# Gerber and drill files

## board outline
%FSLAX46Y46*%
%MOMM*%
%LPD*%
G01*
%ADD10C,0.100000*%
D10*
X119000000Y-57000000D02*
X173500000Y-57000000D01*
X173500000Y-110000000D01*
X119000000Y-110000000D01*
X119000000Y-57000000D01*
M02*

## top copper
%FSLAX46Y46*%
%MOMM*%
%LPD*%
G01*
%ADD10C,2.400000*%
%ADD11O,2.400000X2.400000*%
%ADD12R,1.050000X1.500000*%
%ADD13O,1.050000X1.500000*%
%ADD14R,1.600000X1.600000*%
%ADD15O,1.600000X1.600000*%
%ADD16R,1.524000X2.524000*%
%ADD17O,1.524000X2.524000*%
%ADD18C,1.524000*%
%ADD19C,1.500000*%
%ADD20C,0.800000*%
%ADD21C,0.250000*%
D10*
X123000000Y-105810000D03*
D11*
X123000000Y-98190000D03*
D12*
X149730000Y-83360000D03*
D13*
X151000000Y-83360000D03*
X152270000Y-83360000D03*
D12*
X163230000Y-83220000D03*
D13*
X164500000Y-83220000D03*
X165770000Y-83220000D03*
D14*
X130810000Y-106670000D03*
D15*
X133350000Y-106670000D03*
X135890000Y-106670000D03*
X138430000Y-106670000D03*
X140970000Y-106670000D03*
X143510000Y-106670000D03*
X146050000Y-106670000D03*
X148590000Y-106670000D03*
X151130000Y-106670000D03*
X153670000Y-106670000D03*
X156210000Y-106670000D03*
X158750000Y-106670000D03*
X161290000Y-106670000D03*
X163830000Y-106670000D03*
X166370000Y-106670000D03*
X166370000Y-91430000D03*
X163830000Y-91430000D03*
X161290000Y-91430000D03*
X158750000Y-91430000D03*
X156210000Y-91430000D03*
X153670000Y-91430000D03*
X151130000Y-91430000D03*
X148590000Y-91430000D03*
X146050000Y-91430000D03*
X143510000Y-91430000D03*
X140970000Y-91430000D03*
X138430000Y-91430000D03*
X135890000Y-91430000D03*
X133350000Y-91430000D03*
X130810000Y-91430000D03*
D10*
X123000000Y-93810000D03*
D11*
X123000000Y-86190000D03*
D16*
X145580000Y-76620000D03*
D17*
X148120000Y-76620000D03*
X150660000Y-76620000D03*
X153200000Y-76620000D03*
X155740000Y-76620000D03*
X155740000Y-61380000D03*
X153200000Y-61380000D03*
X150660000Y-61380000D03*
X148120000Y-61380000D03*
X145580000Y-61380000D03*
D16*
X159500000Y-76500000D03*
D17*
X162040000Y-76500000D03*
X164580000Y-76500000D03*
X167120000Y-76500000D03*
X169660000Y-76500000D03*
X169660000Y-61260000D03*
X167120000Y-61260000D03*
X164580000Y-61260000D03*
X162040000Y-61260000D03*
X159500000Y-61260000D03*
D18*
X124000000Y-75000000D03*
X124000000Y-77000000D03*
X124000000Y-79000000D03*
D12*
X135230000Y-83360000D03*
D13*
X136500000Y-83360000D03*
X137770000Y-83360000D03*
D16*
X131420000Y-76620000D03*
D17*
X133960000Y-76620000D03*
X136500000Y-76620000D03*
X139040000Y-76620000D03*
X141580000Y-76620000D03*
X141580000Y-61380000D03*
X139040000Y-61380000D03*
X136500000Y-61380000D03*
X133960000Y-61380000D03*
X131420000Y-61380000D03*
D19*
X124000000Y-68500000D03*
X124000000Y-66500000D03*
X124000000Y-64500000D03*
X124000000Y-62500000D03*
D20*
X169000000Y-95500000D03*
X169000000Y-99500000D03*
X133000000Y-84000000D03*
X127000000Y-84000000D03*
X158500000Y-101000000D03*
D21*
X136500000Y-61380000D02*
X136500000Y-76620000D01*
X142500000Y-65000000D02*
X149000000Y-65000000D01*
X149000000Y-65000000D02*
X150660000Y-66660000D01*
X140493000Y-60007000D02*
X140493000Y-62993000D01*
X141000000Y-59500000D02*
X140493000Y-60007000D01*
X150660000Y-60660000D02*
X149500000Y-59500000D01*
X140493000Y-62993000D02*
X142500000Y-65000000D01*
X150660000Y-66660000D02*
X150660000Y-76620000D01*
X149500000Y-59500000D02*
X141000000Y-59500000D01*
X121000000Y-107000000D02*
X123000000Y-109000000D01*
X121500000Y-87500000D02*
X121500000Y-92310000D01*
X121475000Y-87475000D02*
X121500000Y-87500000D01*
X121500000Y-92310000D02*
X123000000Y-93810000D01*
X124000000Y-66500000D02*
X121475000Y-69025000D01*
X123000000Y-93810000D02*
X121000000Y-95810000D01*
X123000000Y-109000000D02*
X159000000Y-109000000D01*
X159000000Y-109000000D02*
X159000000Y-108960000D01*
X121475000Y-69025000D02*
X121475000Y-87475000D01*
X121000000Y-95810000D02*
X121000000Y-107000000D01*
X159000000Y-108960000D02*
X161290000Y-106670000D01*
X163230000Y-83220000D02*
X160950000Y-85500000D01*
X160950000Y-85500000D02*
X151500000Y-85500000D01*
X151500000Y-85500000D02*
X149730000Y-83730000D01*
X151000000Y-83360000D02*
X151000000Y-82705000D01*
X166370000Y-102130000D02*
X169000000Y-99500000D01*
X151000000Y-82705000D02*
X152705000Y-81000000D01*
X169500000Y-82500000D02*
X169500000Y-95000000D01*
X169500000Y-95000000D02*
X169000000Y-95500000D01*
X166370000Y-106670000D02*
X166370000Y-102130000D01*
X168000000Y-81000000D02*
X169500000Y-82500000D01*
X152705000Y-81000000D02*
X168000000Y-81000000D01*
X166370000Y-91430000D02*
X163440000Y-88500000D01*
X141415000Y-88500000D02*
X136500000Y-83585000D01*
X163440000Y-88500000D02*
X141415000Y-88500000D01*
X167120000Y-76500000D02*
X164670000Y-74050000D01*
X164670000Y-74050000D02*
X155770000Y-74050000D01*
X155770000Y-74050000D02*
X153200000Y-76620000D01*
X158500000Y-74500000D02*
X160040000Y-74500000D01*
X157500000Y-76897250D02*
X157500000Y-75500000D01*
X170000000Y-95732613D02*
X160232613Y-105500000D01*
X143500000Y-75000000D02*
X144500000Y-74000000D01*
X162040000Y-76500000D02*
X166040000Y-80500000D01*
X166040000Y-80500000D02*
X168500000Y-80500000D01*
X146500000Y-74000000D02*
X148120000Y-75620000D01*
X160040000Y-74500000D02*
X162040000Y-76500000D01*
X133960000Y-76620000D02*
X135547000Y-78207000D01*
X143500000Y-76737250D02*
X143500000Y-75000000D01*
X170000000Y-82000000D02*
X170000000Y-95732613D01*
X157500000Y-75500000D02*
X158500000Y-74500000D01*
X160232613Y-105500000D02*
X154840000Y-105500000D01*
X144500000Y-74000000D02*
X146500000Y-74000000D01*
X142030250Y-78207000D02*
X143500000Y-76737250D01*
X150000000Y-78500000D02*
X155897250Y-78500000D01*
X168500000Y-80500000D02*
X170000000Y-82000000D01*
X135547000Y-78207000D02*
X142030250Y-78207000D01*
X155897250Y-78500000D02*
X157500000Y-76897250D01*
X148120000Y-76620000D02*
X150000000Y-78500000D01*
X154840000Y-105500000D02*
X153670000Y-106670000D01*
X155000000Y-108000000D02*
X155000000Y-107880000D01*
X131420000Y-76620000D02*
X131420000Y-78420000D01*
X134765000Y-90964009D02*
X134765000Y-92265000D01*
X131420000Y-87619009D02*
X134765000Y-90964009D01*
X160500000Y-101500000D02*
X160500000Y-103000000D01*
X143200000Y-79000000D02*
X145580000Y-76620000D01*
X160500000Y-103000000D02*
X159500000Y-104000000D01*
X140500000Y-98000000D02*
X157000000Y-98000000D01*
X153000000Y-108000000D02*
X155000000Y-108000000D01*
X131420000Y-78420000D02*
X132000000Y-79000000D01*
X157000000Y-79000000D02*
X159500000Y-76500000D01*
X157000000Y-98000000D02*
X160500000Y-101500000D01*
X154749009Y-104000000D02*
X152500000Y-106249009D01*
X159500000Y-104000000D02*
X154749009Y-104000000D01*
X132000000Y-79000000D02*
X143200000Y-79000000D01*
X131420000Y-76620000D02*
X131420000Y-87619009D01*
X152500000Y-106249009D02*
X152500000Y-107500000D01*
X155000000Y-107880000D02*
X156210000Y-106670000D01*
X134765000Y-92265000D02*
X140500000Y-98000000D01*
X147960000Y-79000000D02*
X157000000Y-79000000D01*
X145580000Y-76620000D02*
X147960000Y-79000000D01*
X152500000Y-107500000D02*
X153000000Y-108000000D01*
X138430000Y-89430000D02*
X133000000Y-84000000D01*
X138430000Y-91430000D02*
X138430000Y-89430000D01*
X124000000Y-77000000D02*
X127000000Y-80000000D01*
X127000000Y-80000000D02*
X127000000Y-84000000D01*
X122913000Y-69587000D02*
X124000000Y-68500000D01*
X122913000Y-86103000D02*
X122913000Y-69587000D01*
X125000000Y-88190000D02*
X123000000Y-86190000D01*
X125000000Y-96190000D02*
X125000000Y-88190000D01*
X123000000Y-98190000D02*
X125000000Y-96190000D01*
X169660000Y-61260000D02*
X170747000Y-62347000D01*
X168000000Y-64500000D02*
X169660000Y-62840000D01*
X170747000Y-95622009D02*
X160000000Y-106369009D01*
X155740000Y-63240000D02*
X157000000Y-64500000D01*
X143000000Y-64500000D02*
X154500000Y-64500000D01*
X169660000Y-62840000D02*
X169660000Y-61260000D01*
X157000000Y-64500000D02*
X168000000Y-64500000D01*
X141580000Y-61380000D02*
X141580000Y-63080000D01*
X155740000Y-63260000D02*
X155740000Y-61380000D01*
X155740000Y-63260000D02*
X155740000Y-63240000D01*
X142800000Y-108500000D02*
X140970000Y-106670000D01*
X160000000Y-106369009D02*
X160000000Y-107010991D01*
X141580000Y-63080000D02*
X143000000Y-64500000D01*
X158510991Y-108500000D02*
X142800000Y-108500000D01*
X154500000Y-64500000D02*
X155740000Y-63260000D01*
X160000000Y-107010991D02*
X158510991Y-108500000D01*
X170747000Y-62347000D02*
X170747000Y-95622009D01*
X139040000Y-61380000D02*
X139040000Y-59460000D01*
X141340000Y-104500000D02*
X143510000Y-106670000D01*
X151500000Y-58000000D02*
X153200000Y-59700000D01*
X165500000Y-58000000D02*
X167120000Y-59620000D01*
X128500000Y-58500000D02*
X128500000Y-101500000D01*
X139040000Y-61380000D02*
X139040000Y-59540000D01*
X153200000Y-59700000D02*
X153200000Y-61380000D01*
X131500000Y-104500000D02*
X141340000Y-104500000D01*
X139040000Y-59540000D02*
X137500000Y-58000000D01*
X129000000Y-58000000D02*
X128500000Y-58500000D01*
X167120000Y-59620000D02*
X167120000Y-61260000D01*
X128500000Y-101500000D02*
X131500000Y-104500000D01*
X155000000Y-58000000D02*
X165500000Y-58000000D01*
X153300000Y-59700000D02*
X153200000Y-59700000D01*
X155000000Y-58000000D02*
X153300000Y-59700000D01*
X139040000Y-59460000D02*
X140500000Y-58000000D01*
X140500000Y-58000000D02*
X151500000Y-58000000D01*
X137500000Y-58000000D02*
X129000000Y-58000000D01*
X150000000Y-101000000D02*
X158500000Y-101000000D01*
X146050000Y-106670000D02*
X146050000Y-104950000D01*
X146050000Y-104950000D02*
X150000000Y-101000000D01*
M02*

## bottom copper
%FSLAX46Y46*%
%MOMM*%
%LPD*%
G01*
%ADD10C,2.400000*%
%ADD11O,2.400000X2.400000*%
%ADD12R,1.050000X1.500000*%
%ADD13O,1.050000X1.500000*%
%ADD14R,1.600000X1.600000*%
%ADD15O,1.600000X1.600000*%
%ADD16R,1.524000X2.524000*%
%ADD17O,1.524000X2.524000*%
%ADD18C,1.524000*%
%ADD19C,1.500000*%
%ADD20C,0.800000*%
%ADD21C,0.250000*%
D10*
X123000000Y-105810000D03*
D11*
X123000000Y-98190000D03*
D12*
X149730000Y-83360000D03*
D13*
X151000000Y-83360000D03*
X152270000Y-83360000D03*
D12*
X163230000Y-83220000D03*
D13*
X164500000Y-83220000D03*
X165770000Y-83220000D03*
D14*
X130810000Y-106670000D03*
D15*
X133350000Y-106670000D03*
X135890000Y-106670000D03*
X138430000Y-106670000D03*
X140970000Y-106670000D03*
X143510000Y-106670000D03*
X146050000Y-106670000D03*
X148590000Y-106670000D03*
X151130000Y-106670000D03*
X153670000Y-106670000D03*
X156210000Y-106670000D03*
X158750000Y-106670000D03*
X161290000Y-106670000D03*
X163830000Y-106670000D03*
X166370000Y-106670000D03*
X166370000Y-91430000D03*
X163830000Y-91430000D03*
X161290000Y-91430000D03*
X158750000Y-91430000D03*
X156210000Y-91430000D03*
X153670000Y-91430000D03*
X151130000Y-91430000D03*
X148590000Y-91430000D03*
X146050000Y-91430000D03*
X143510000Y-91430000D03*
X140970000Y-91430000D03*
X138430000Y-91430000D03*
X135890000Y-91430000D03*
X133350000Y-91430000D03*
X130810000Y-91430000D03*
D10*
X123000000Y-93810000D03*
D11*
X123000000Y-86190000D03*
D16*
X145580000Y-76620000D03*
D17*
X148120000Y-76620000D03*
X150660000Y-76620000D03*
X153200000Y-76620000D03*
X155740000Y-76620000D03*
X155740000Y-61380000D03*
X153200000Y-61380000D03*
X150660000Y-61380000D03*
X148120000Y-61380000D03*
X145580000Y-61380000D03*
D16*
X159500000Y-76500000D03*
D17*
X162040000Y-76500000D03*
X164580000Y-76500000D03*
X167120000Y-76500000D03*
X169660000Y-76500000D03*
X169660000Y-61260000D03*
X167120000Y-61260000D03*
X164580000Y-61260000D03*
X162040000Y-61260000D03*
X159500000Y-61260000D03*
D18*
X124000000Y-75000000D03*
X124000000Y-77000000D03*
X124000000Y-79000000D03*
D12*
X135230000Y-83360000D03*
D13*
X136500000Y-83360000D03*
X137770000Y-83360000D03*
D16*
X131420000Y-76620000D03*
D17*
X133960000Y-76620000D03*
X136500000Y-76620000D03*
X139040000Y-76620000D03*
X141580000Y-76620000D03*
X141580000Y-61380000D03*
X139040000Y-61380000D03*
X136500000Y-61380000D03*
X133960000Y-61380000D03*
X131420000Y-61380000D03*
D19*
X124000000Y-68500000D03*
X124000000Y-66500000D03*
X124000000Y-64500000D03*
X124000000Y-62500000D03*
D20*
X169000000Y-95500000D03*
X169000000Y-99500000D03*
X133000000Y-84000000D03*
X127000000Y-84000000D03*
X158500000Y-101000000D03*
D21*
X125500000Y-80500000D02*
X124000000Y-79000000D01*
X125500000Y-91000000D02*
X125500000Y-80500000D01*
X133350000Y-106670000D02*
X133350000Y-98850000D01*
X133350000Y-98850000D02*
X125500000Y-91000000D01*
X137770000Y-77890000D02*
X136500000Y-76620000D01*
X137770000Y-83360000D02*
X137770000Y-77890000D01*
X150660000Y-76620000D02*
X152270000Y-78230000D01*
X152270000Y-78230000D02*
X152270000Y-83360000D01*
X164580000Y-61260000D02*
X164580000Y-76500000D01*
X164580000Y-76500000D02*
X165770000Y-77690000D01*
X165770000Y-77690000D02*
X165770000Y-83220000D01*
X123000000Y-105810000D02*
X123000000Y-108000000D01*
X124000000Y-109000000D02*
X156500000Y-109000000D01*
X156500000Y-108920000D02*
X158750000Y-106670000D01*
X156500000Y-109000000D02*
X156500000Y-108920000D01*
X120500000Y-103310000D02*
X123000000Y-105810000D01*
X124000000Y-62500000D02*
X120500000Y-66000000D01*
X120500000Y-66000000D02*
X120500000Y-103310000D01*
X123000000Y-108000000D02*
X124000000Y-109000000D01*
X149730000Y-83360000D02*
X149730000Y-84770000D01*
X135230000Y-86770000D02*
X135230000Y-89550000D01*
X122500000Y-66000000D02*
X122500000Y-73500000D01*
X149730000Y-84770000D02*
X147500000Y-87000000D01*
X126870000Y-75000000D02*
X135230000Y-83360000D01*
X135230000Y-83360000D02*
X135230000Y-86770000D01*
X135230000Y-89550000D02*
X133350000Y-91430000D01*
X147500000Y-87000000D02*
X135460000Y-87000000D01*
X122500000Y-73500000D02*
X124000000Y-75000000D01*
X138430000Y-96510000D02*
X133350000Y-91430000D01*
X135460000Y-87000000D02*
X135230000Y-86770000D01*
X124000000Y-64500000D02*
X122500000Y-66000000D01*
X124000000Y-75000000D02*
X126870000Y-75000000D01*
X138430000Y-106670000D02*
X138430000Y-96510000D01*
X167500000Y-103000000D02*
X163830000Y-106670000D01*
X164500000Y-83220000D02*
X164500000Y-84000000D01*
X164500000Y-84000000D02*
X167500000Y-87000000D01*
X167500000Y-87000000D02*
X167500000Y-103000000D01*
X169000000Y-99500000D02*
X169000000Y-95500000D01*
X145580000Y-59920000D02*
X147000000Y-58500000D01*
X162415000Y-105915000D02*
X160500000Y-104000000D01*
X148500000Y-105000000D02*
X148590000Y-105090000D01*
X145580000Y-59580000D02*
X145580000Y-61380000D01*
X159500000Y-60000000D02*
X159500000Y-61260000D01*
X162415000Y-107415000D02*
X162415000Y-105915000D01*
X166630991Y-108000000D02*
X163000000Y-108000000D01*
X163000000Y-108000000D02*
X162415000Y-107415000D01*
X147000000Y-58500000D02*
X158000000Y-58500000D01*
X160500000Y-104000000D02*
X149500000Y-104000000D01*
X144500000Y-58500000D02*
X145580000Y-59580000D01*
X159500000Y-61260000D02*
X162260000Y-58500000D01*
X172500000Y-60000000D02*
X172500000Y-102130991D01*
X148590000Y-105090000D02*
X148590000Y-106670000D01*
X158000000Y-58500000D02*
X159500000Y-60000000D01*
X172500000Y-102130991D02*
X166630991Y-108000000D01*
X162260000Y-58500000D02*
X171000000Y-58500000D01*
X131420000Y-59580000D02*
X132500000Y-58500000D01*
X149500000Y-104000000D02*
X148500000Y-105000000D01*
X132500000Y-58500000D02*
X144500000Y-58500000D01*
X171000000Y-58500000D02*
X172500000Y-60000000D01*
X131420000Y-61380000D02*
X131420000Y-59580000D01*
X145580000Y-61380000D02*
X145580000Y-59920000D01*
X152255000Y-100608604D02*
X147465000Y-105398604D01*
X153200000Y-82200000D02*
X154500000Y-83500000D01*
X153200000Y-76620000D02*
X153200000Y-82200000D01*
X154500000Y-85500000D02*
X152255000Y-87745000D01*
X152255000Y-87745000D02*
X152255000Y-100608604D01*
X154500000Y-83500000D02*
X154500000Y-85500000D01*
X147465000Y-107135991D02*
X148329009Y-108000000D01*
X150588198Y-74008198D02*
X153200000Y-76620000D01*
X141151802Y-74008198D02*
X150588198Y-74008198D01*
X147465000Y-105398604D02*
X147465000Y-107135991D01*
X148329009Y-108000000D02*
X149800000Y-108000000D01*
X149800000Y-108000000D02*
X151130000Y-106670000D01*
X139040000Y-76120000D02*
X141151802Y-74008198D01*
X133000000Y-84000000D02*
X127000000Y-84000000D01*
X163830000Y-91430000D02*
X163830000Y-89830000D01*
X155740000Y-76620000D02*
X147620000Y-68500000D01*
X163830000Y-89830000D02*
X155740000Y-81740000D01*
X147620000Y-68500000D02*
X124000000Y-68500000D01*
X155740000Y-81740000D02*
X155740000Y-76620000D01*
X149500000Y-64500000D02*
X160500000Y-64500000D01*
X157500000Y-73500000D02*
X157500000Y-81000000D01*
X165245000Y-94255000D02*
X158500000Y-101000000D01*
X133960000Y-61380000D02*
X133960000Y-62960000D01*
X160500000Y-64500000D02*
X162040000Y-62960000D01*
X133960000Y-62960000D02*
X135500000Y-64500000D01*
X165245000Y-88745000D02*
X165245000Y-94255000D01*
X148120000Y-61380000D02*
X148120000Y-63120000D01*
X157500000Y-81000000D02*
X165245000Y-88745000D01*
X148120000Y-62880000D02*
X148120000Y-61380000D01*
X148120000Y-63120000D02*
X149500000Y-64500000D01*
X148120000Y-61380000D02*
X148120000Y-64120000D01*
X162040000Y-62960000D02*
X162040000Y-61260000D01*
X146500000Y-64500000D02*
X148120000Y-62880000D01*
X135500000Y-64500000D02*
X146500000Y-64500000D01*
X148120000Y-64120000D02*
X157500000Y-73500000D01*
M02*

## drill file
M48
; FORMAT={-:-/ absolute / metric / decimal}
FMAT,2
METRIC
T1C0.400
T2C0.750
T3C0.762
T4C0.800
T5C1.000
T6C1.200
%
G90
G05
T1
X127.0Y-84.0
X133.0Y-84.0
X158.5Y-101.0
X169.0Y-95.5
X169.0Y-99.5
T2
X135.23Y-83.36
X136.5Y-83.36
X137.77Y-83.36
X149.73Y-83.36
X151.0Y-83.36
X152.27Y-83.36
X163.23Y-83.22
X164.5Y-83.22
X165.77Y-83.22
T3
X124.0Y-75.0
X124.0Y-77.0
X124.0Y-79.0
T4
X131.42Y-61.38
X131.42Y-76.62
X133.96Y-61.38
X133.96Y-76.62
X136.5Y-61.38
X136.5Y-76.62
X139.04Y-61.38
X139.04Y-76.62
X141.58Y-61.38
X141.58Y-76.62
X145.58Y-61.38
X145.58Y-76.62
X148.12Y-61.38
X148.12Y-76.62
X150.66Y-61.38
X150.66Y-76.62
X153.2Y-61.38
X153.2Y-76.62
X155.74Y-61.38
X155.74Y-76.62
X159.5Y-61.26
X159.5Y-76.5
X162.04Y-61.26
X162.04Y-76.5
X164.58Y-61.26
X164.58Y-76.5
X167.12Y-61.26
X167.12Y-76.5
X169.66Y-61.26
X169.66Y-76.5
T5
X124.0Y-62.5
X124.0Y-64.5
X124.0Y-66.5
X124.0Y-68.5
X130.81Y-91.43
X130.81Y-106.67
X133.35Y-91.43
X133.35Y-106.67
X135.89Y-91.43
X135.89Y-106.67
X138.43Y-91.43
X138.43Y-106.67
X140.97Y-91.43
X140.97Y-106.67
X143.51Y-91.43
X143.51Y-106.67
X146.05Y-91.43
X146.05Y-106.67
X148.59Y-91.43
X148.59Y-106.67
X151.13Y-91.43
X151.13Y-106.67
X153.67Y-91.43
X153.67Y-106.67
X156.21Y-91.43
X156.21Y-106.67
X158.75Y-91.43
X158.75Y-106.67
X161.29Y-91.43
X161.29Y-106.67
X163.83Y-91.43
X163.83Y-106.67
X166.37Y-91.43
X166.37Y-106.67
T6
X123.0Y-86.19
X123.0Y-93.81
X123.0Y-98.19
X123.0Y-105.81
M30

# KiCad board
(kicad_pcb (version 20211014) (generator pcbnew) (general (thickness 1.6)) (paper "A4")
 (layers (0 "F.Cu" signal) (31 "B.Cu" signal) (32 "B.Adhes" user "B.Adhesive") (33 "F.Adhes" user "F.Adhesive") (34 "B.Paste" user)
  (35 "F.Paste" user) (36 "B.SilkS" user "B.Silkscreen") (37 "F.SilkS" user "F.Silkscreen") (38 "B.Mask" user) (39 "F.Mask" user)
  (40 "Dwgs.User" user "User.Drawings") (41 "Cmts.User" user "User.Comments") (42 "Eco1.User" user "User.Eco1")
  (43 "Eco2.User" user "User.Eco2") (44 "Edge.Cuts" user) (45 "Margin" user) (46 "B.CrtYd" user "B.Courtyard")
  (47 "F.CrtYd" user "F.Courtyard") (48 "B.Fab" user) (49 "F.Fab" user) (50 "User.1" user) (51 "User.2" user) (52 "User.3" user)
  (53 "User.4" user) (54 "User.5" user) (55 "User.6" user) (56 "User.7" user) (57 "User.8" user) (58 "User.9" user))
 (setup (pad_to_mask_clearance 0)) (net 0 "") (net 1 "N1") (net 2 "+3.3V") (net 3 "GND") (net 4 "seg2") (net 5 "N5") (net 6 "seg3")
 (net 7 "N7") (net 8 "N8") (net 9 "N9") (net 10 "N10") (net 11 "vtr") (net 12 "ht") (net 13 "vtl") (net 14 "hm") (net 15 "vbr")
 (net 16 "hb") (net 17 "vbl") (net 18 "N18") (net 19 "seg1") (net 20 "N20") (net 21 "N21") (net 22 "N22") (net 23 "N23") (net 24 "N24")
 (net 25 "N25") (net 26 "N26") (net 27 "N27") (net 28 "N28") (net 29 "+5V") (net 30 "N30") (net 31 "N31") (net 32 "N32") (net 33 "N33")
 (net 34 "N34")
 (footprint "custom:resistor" (layer "F.Cu") (at 123 105.81 90)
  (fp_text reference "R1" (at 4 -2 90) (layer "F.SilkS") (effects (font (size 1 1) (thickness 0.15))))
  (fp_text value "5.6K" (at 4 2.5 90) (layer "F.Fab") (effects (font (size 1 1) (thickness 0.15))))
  (pad "1" thru_hole circle (at 0 0 90) (size 2.4 2.4) (drill 1.2) (layers *.Cu *.Mask) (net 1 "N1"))
  (pad "2" thru_hole oval (at 7.62 0 90) (size 2.4 2.4) (drill 1.2) (layers *.Cu *.Mask) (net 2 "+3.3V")))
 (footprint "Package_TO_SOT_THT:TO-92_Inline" (layer "F.Cu") (at 149.73 83.36)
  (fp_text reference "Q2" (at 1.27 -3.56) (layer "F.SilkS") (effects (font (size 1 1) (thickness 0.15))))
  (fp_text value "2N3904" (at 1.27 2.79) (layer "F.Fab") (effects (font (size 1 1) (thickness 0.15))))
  (pad "1" thru_hole rect (at 0 0) (size 1.05 1.5) (drill 0.75) (layers *.Cu *.Mask) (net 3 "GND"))
  (pad "2" thru_hole oval (at 1.27 0) (size 1.05 1.5) (drill 0.75) (layers *.Cu *.Mask) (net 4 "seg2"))
  (pad "3" thru_hole oval (at 2.54 0) (size 1.05 1.5) (drill 0.75) (layers *.Cu *.Mask) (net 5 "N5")))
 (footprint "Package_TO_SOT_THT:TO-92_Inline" (layer "F.Cu") (at 163.23 83.22)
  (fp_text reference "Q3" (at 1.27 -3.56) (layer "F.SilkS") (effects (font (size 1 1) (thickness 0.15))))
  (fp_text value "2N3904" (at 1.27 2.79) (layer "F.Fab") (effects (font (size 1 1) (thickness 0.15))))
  (pad "1" thru_hole rect (at 0 0) (size 1.05 1.5) (drill 0.75) (layers *.Cu *.Mask) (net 3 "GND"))
  (pad "2" thru_hole oval (at 1.27 0) (size 1.05 1.5) (drill 0.75) (layers *.Cu *.Mask) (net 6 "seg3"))
  (pad "3" thru_hole oval (at 2.54 0) (size 1.05 1.5) (drill 0.75) (layers *.Cu *.Mask) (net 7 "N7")))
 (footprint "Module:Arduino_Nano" (layer "F.Cu") (at 130.81 106.67 90)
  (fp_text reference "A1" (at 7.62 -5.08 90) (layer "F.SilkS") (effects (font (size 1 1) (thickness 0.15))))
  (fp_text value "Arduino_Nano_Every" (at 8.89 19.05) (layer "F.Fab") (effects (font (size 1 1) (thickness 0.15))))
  (pad "1" thru_hole rect (at 0 0 90) (size 1.6 1.6) (drill 1) (layers *.Cu *.Mask) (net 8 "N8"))
  (pad "2" thru_hole oval (at 0 2.54 90) (size 1.6 1.6) (drill 1) (layers *.Cu *.Mask) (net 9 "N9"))
  (pad "3" thru_hole oval (at 0 5.08 90) (size 1.6 1.6) (drill 1) (layers *.Cu *.Mask) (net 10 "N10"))
  (pad "4" thru_hole oval (at 0 7.62 90) (size 1.6 1.6) (drill 1) (layers *.Cu *.Mask) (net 3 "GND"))
  (pad "5" thru_hole oval (at 0 10.16 90) (size 1.6 1.6) (drill 1) (layers *.Cu *.Mask) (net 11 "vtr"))
  (pad "6" thru_hole oval (at 0 12.7 90) (size 1.6 1.6) (drill 1) (layers *.Cu *.Mask) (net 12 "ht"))
  (pad "7" thru_hole oval (at 0 15.24 90) (size 1.6 1.6) (drill 1) (layers *.Cu *.Mask) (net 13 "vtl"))
  (pad "8" thru_hole oval (at 0 17.78 90) (size 1.6 1.6) (drill 1) (layers *.Cu *.Mask) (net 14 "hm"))
  (pad "9" thru_hole oval (at 0 20.32 90) (size 1.6 1.6) (drill 1) (layers *.Cu *.Mask) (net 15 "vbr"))
  (pad "10" thru_hole oval (at 0 22.86 90) (size 1.6 1.6) (drill 1) (layers *.Cu *.Mask) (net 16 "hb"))
  (pad "11" thru_hole oval (at 0 25.4 90) (size 1.6 1.6) (drill 1) (layers *.Cu *.Mask) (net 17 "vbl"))
  (pad "12" thru_hole oval (at 0 27.94 90) (size 1.6 1.6) (drill 1) (layers *.Cu *.Mask) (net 1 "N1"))
  (pad "13" thru_hole oval (at 0 30.48 90) (size 1.6 1.6) (drill 1) (layers *.Cu *.Mask) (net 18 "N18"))
  (pad "14" thru_hole oval (at 0 33.02 90) (size 1.6 1.6) (drill 1) (layers *.Cu *.Mask) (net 6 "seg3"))
  (pad "15" thru_hole oval (at 0 35.56 90) (size 1.6 1.6) (drill 1) (layers *.Cu *.Mask) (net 4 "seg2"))
  (pad "16" thru_hole oval (at 15.24 35.56 90) (size 1.6 1.6) (drill 1) (layers *.Cu *.Mask) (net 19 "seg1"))
  (pad "17" thru_hole oval (at 15.24 33.02 90) (size 1.6 1.6) (drill 1) (layers *.Cu *.Mask) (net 2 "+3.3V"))
  (pad "18" thru_hole oval (at 15.24 30.48 90) (size 1.6 1.6) (drill 1) (layers *.Cu *.Mask) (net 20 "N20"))
  (pad "19" thru_hole oval (at 15.24 27.94 90) (size 1.6 1.6) (drill 1) (layers *.Cu *.Mask) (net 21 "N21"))
  (pad "20" thru_hole oval (at 15.24 25.4 90) (size 1.6 1.6) (drill 1) (layers *.Cu *.Mask) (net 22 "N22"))
  (pad "21" thru_hole oval (at 15.24 22.86 90) (size 1.6 1.6) (drill 1) (layers *.Cu *.Mask) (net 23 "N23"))
  (pad "22" thru_hole oval (at 15.24 20.32 90) (size 1.6 1.6) (drill 1) (layers *.Cu *.Mask) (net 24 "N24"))
  (pad "23" thru_hole oval (at 15.24 17.78 90) (size 1.6 1.6) (drill 1) (layers *.Cu *.Mask) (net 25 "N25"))
  (pad "24" thru_hole oval (at 15.24 15.24 90) (size 1.6 1.6) (drill 1) (layers *.Cu *.Mask) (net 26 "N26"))
  (pad "25" thru_hole oval (at 15.24 12.7 90) (size 1.6 1.6) (drill 1) (layers *.Cu *.Mask) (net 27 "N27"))
  (pad "26" thru_hole oval (at 15.24 10.16 90) (size 1.6 1.6) (drill 1) (layers *.Cu *.Mask) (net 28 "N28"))
  (pad "27" thru_hole oval (at 15.24 7.62 90) (size 1.6 1.6) (drill 1) (layers *.Cu *.Mask) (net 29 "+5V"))
  (pad "28" thru_hole oval (at 15.24 5.08 90) (size 1.6 1.6) (drill 1) (layers *.Cu *.Mask) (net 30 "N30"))
  (pad "29" thru_hole oval (at 15.24 2.54 90) (size 1.6 1.6) (drill 1) (layers *.Cu *.Mask) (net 3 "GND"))
  (pad "30" thru_hole oval (at 15.24 0 90) (size 1.6 1.6) (drill 1) (layers *.Cu *.Mask) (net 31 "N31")))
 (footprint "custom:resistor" (layer "F.Cu") (at 123 93.81 90)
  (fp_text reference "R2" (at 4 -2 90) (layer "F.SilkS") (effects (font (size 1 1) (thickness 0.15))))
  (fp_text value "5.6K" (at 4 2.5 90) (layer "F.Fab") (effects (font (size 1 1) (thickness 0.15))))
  (pad "1" thru_hole circle (at 0 0 90) (size 2.4 2.4) (drill 1.2) (layers *.Cu *.Mask) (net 18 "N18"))
  (pad "2" thru_hole oval (at 7.62 0 90) (size 2.4 2.4) (drill 1.2) (layers *.Cu *.Mask) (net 2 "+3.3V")))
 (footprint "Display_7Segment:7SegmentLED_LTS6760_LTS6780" (layer "F.Cu") (at 145.58 76.62 90)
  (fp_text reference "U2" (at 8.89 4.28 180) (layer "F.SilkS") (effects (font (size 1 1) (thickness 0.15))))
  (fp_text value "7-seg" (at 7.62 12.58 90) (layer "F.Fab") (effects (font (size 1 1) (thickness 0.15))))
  (pad "1" thru_hole rect (at 0 0) (size 1.524 2.524) (drill 0.8) (layers *.Cu *.Mask) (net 17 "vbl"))
  (pad "2" thru_hole oval (at 0 2.54) (size 1.524 2.524) (drill 0.8) (layers *.Cu *.Mask) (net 16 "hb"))
  (pad "3" thru_hole oval (at 0 5.08) (size 1.524 2.524) (drill 0.8) (layers *.Cu *.Mask) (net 5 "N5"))
  (pad "4" thru_hole oval (at 0 7.62) (size 1.524 2.524) (drill 0.8) (layers *.Cu *.Mask) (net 15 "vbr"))
  (pad "5" thru_hole oval (at 0 10.16) (size 1.524 2.524) (drill 0.8) (layers *.Cu *.Mask) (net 2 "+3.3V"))
  (pad "6" thru_hole oval (at 15.24 10.16) (size 1.524 2.524) (drill 0.8) (layers *.Cu *.Mask) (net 11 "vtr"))
  (pad "7" thru_hole oval (at 15.24 7.62) (size 1.524 2.524) (drill 0.8) (layers *.Cu *.Mask) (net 12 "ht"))
  (pad "8" thru_hole oval (at 15.24 5.08) (size 1.524 2.524) (drill 0.8) (layers *.Cu *.Mask) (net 5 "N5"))
  (pad "9" thru_hole oval (at 15.24 2.54) (size 1.524 2.524) (drill 0.8) (layers *.Cu *.Mask) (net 13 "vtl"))
  (pad "10" thru_hole oval (at 15.24 0) (size 1.524 2.524) (drill 0.8) (layers *.Cu *.Mask) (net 14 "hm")))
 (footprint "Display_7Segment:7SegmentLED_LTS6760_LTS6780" (layer "F.Cu") (at 159.5 76.5 90)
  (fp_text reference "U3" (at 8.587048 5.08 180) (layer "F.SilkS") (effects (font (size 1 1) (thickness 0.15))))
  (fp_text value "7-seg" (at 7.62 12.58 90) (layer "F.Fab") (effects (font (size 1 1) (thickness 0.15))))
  (pad "1" thru_hole rect (at 0 0) (size 1.524 2.524) (drill 0.8) (layers *.Cu *.Mask) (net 17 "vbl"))
  (pad "2" thru_hole oval (at 0 2.54) (size 1.524 2.524) (drill 0.8) (layers *.Cu *.Mask) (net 16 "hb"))
  (pad "3" thru_hole oval (at 0 5.08) (size 1.524 2.524) (drill 0.8) (layers *.Cu *.Mask) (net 7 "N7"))
  (pad "4" thru_hole oval (at 0 7.62) (size 1.524 2.524) (drill 0.8) (layers *.Cu *.Mask) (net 15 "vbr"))
  (pad "5" thru_hole oval (at 0 10.16) (size 1.524 2.524) (drill 0.8) (layers *.Cu *.Mask) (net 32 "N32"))
  (pad "6" thru_hole oval (at 15.24 10.16) (size 1.524 2.524) (drill 0.8) (layers *.Cu *.Mask) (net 11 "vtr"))
  (pad "7" thru_hole oval (at 15.24 7.62) (size 1.524 2.524) (drill 0.8) (layers *.Cu *.Mask) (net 12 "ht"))
  (pad "8" thru_hole oval (at 15.24 5.08) (size 1.524 2.524) (drill 0.8) (layers *.Cu *.Mask) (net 7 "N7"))
  (pad "9" thru_hole oval (at 15.24 2.54) (size 1.524 2.524) (drill 0.8) (layers *.Cu *.Mask) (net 13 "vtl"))
  (pad "10" thru_hole oval (at 15.24 0) (size 1.524 2.524) (drill 0.8) (layers *.Cu *.Mask) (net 14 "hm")))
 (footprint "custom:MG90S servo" (layer "F.Cu") (at 124 77 -90)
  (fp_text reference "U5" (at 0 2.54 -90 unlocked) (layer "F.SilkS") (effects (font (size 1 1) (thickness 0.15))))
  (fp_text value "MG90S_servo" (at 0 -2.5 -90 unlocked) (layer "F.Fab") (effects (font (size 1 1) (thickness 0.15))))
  (pad "1" thru_hole circle (at -2 0 270) (size 1.524 1.524) (drill 0.762) (layers *.Cu *.Mask) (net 3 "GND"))
  (pad "2" thru_hole circle (at 0 0 270) (size 1.524 1.524) (drill 0.762) (layers *.Cu *.Mask) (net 29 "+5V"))
  (pad "3" thru_hole circle (at 2 0 270) (size 1.524 1.524) (drill 0.762) (layers *.Cu *.Mask) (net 9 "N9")))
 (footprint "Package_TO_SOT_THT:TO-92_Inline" (layer "F.Cu") (at 135.23 83.36)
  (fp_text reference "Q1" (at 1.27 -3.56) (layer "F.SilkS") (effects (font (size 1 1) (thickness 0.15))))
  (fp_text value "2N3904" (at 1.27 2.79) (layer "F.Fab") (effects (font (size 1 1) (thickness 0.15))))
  (pad "1" thru_hole rect (at 0 0) (size 1.05 1.5) (drill 0.75) (layers *.Cu *.Mask) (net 3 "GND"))
  (pad "2" thru_hole oval (at 1.27 0) (size 1.05 1.5) (drill 0.75) (layers *.Cu *.Mask) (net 19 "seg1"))
  (pad "3" thru_hole oval (at 2.54 0) (size 1.05 1.5) (drill 0.75) (layers *.Cu *.Mask) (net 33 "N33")))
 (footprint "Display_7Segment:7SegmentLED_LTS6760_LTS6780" (layer "F.Cu") (at 131.42 76.62 90)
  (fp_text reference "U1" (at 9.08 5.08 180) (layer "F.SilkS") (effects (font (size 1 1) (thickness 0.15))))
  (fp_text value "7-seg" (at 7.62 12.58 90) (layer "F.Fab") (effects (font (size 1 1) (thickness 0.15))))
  (pad "1" thru_hole rect (at 0 0) (size 1.524 2.524) (drill 0.8) (layers *.Cu *.Mask) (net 17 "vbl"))
  (pad "2" thru_hole oval (at 0 2.54) (size 1.524 2.524) (drill 0.8) (layers *.Cu *.Mask) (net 16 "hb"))
  (pad "3" thru_hole oval (at 0 5.08) (size 1.524 2.524) (drill 0.8) (layers *.Cu *.Mask) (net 33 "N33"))
  (pad "4" thru_hole oval (at 0 7.62) (size 1.524 2.524) (drill 0.8) (layers *.Cu *.Mask) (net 15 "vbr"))
  (pad "5" thru_hole oval (at 0 10.16) (size 1.524 2.524) (drill 0.8) (layers *.Cu *.Mask) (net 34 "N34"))
  (pad "6" thru_hole oval (at 15.24 10.16) (size 1.524 2.524) (drill 0.8) (layers *.Cu *.Mask) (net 11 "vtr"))
  (pad "7" thru_hole oval (at 15.24 7.62) (size 1.524 2.524) (drill 0.8) (layers *.Cu *.Mask) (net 12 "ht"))
  (pad "8" thru_hole oval (at 15.24 5.08) (size 1.524 2.524) (drill 0.8) (layers *.Cu *.Mask) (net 33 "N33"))
  (pad "9" thru_hole oval (at 15.24 2.54) (size 1.524 2.524) (drill 0.8) (layers *.Cu *.Mask) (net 13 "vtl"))
  (pad "10" thru_hole oval (at 15.24 0) (size 1.524 2.524) (drill 0.8) (layers *.Cu *.Mask) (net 14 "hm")))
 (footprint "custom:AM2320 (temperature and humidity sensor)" (layer "F.Cu") (at 124 65.5 90)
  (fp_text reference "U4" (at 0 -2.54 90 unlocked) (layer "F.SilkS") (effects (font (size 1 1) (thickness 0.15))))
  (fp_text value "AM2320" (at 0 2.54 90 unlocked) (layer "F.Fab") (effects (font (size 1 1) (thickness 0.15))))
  (pad "1" thru_hole circle (at -3 0 90) (size 1.5 1.5) (drill 1) (layers *.Cu *.Mask) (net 2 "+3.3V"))
  (pad "2" thru_hole circle (at -1 0 90) (size 1.5 1.5) (drill 1) (layers *.Cu *.Mask) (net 18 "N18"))
  (pad "3" thru_hole circle (at 1 0 90) (size 1.5 1.5) (drill 1) (layers *.Cu *.Mask) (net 3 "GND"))
  (pad "4" thru_hole circle (at 3 0 90) (size 1.5 1.5) (drill 1) (layers *.Cu *.Mask) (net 1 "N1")))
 (gr_rect (start 173.5 57) (end 119 110) (layer "Edge.Cuts") (width 0.1) (fill none))
 (segment (start 125.5 80.5) (end 124 79) (width 0.25) (layer "B.Cu") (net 9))
 (segment (start 125.5 91) (end 125.5 80.5) (width 0.25) (layer "B.Cu") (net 9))
 (segment (start 133.35 106.67) (end 133.35 98.85) (width 0.25) (layer "B.Cu") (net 9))
 (segment (start 133.35 98.85) (end 125.5 91) (width 0.25) (layer "B.Cu") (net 9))
 (segment (start 136.5 61.38) (end 136.5 76.62) (width 0.25) (layer "F.Cu") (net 33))
 (segment (start 137.77 77.89) (end 136.5 76.62) (width 0.25) (layer "B.Cu") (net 33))
 (segment (start 137.77 83.36) (end 137.77 77.89) (width 0.25) (layer "B.Cu") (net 33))
 (segment (start 142.5 65) (end 149 65) (width 0.25) (layer "F.Cu") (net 5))
 (segment (start 149 65) (end 150.66 66.66) (width 0.25) (layer "F.Cu") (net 5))
 (segment (start 140.493 60.007) (end 140.493 62.993) (width 0.25) (layer "F.Cu") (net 5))
 (segment (start 141 59.5) (end 140.493 60.007) (width 0.25) (layer "F.Cu") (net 5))
 (segment (start 150.66 60.66) (end 149.5 59.5) (width 0.25) (layer "F.Cu") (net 5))
 (segment (start 140.493 62.993) (end 142.5 65) (width 0.25) (layer "F.Cu") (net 5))
 (segment (start 150.66 66.66) (end 150.66 76.62) (width 0.25) (layer "F.Cu") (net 5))
 (segment (start 149.5 59.5) (end 141 59.5) (width 0.25) (layer "F.Cu") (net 5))
 (segment (start 150.66 76.62) (end 152.27 78.23) (width 0.25) (layer "B.Cu") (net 5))
 (segment (start 152.27 78.23) (end 152.27 83.36) (width 0.25) (layer "B.Cu") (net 5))
 (segment (start 164.58 61.26) (end 164.58 76.5) (width 0.25) (layer "B.Cu") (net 7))
 (segment (start 164.58 76.5) (end 165.77 77.69) (width 0.25) (layer "B.Cu") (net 7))
 (segment (start 165.77 77.69) (end 165.77 83.22) (width 0.25) (layer "B.Cu") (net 7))
 (segment (start 123 105.81) (end 123 108) (width 0.25) (layer "B.Cu") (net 1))
 (segment (start 124 109) (end 156.5 109) (width 0.25) (layer "B.Cu") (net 1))
 (segment (start 156.5 108.92) (end 158.75 106.67) (width 0.25) (layer "B.Cu") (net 1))
 (segment (start 156.5 109) (end 156.5 108.92) (width 0.25) (layer "B.Cu") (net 1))
 (segment (start 120.5 103.31) (end 123 105.81) (width 0.25) (layer "B.Cu") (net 1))
 (segment (start 124 62.5) (end 120.5 66) (width 0.25) (layer "B.Cu") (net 1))
 (segment (start 120.5 66) (end 120.5 103.31) (width 0.25) (layer "B.Cu") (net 1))
 (segment (start 123 108) (end 124 109) (width 0.25) (layer "B.Cu") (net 1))
 (segment (start 121 107) (end 123 109) (width 0.25) (layer "F.Cu") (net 18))
 (segment (start 121.5 87.5) (end 121.5 92.31) (width 0.25) (layer "F.Cu") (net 18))
 (segment (start 121.475 87.475) (end 121.5 87.5) (width 0.25) (layer "F.Cu") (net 18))
 (segment (start 121.5 92.31) (end 123 93.81) (width 0.25) (layer "F.Cu") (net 18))
 (segment (start 124 66.5) (end 121.475 69.025) (width 0.25) (layer "F.Cu") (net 18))
 (segment (start 123 93.81) (end 121 95.81) (width 0.25) (layer "F.Cu") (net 18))
 (segment (start 123 109) (end 159 109) (width 0.25) (layer "F.Cu") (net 18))
 (segment (start 159 109) (end 159 108.96) (width 0.25) (layer "F.Cu") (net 18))
 (segment (start 121.475 69.025) (end 121.475 87.475) (width 0.25) (layer "F.Cu") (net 18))
 (segment (start 121 95.81) (end 121 107) (width 0.25) (layer "F.Cu") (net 18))
 (segment (start 159 108.96) (end 161.29 106.67) (width 0.25) (layer "F.Cu") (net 18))
 (segment (start 163.23 83.22) (end 160.95 85.5) (width 0.25) (layer "F.Cu") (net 3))
 (segment (start 160.95 85.5) (end 151.5 85.5) (width 0.25) (layer "F.Cu") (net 3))
 (segment (start 151.5 85.5) (end 149.73 83.73) (width 0.25) (layer "F.Cu") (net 3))
 (segment (start 149.73 83.36) (end 149.73 84.77) (width 0.25) (layer "B.Cu") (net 3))
 (segment (start 135.23 86.77) (end 135.23 89.55) (width 0.25) (layer "B.Cu") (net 3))
 (segment (start 122.5 66) (end 122.5 73.5) (width 0.25) (layer "B.Cu") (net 3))
 (segment (start 149.73 84.77) (end 147.5 87) (width 0.25) (layer "B.Cu") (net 3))
 (segment (start 126.87 75) (end 135.23 83.36) (width 0.25) (layer "B.Cu") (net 3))
 (segment (start 135.23 83.36) (end 135.23 86.77) (width 0.25) (layer "B.Cu") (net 3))
 (segment (start 135.23 89.55) (end 133.35 91.43) (width 0.25) (layer "B.Cu") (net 3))
 (segment (start 147.5 87) (end 135.46 87) (width 0.25) (layer "B.Cu") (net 3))
 (segment (start 122.5 73.5) (end 124 75) (width 0.25) (layer "B.Cu") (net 3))
 (segment (start 138.43 96.51) (end 133.35 91.43) (width 0.25) (layer "B.Cu") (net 3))
 (segment (start 135.46 87) (end 135.23 86.77) (width 0.25) (layer "B.Cu") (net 3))
 (segment (start 124 64.5) (end 122.5 66) (width 0.25) (layer "B.Cu") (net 3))
 (segment (start 124 75) (end 126.87 75) (width 0.25) (layer "B.Cu") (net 3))
 (segment (start 138.43 106.67) (end 138.43 96.51) (width 0.25) (layer "B.Cu") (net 3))
 (segment (start 167.5 103) (end 163.83 106.67) (width 0.25) (layer "B.Cu") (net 6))
 (segment (start 164.5 83.22) (end 164.5 84) (width 0.25) (layer "B.Cu") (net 6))
 (segment (start 164.5 84) (end 167.5 87) (width 0.25) (layer "B.Cu") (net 6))
 (segment (start 167.5 87) (end 167.5 103) (width 0.25) (layer "B.Cu") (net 6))
 (segment (start 151 83.36) (end 151 82.705) (width 0.25) (layer "F.Cu") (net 4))
 (segment (start 166.37 102.13) (end 169 99.5) (width 0.25) (layer "F.Cu") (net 4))
 (segment (start 151 82.705) (end 152.705 81) (width 0.25) (layer "F.Cu") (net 4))
 (segment (start 169.5 82.5) (end 169.5 95) (width 0.25) (layer "F.Cu") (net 4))
 (segment (start 169.5 95) (end 169 95.5) (width 0.25) (layer "F.Cu") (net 4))
 (segment (start 166.37 106.67) (end 166.37 102.13) (width 0.25) (layer "F.Cu") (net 4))
 (segment (start 168 81) (end 169.5 82.5) (width 0.25) (layer "F.Cu") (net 4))
 (segment (start 152.705 81) (end 168 81) (width 0.25) (layer "F.Cu") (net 4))
 (via (at 169 95.5) (size 0.8) (drill 0.4) (layers "F.Cu" "B.Cu") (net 4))
 (via (at 169 99.5) (size 0.8) (drill 0.4) (layers "F.Cu" "B.Cu") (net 4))
 (segment (start 169 99.5) (end 169 95.5) (width 0.25) (layer "B.Cu") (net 4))
 (segment (start 166.37 91.43) (end 163.44 88.5) (width 0.25) (layer "F.Cu") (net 19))
 (segment (start 141.415 88.5) (end 136.5 83.585) (width 0.25) (layer "F.Cu") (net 19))
 (segment (start 163.44 88.5) (end 141.415 88.5) (width 0.25) (layer "F.Cu") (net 19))
 (segment (start 145.58 59.92) (end 147 58.5) (width 0.25) (layer "B.Cu") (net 14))
 (segment (start 162.415 105.915) (end 160.5 104) (width 0.25) (layer "B.Cu") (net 14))
 (segment (start 148.5 105) (end 148.59 105.09) (width 0.25) (layer "B.Cu") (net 14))
 (segment (start 145.58 59.58) (end 145.58 61.38) (width 0.25) (layer "B.Cu") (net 14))
 (segment (start 159.5 60) (end 159.5 61.26) (width 0.25) (layer "B.Cu") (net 14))
 (segment (start 162.415 107.415) (end 162.415 105.915) (width 0.25) (layer "B.Cu") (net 14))
 (segment (start 166.630991 108) (end 163 108) (width 0.25) (layer "B.Cu") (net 14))
 (segment (start 163 108) (end 162.415 107.415) (width 0.25) (layer "B.Cu") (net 14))
 (segment (start 147 58.5) (end 158 58.5) (width 0.25) (layer "B.Cu") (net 14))
 (segment (start 160.5 104) (end 149.5 104) (width 0.25) (layer "B.Cu") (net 14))
 (segment (start 144.5 58.5) (end 145.58 59.58) (width 0.25) (layer "B.Cu") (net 14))
 (segment (start 159.5 61.26) (end 162.26 58.5) (width 0.25) (layer "B.Cu") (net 14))
 (segment (start 172.5 60) (end 172.5 102.130991) (width 0.25) (layer "B.Cu") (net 14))
 (segment (start 148.59 105.09) (end 148.59 106.67) (width 0.25) (layer "B.Cu") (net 14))
 (segment (start 158 58.5) (end 159.5 60) (width 0.25) (layer "B.Cu") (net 14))
 (segment (start 172.5 102.130991) (end 166.630991 108) (width 0.25) (layer "B.Cu") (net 14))
 (segment (start 162.26 58.5) (end 171 58.5) (width 0.25) (layer "B.Cu") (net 14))
 (segment (start 131.42 59.58) (end 132.5 58.5) (width 0.25) (layer "B.Cu") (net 14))
 (segment (start 149.5 104) (end 148.5 105) (width 0.25) (layer "B.Cu") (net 14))
 (segment (start 132.5 58.5) (end 144.5 58.5) (width 0.25) (layer "B.Cu") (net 14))
 (segment (start 171 58.5) (end 172.5 60) (width 0.25) (layer "B.Cu") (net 14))
 (segment (start 131.42 61.38) (end 131.42 59.58) (width 0.25) (layer "B.Cu") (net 14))
 (segment (start 145.58 61.38) (end 145.58 59.92) (width 0.25) (layer "B.Cu") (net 14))
 (segment (start 167.12 76.5) (end 164.67 74.05) (width 0.25) (layer "F.Cu") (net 15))
 (segment (start 164.67 74.05) (end 155.77 74.05) (width 0.25) (layer "F.Cu") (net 15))
 (segment (start 155.77 74.05) (end 153.2 76.62) (width 0.25) (layer "F.Cu") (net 15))
 (segment (start 152.255 100.608604) (end 147.465 105.398604) (width 0.25) (layer "B.Cu") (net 15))
 (segment (start 153.2 82.2) (end 154.5 83.5) (width 0.25) (layer "B.Cu") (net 15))
 (segment (start 153.2 76.62) (end 153.2 82.2) (width 0.25) (layer "B.Cu") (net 15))
 (segment (start 154.5 85.5) (end 152.255 87.745) (width 0.25) (layer "B.Cu") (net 15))
 (segment (start 152.255 87.745) (end 152.255 100.608604) (width 0.25) (layer "B.Cu") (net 15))
 (segment (start 154.5 83.5) (end 154.5 85.5) (width 0.25) (layer "B.Cu") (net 15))
 (segment (start 147.465 107.135991) (end 148.329009 108) (width 0.25) (layer "B.Cu") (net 15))
 (segment (start 150.588198 74.008198) (end 153.2 76.62) (width 0.25) (layer "B.Cu") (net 15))
 (segment (start 141.151802 74.008198) (end 150.588198 74.008198) (width 0.25) (layer "B.Cu") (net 15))
 (segment (start 147.465 105.398604) (end 147.465 107.135991) (width 0.25) (layer "B.Cu") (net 15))
 (segment (start 148.329009 108) (end 149.8 108) (width 0.25) (layer "B.Cu") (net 15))
 (segment (start 149.8 108) (end 151.13 106.67) (width 0.25) (layer "B.Cu") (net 15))
 (segment (start 139.04 76.12) (end 141.151802 74.008198) (width 0.25) (layer "B.Cu") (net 15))
 (segment (start 158.5 74.5) (end 160.04 74.5) (width 0.25) (layer "F.Cu") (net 16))
 (segment (start 157.5 76.89725) (end 157.5 75.5) (width 0.25) (layer "F.Cu") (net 16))
 (segment (start 170 95.732613) (end 160.232613 105.5) (width 0.25) (layer "F.Cu") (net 16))
 (segment (start 143.5 75) (end 144.5 74) (width 0.25) (layer "F.Cu") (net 16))
 (segment (start 162.04 76.5) (end 166.04 80.5) (width 0.25) (layer "F.Cu") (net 16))
 (segment (start 166.04 80.5) (end 168.5 80.5) (width 0.25) (layer "F.Cu") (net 16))
 (segment (start 146.5 74) (end 148.12 75.62) (width 0.25) (layer "F.Cu") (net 16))
 (segment (start 160.04 74.5) (end 162.04 76.5) (width 0.25) (layer "F.Cu") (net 16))
 (segment (start 133.96 76.62) (end 135.547 78.207) (width 0.25) (layer "F.Cu") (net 16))
 (segment (start 143.5 76.73725) (end 143.5 75) (width 0.25) (layer "F.Cu") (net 16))
 (segment (start 170 82) (end 170 95.732613) (width 0.25) (layer "F.Cu") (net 16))
 (segment (start 157.5 75.5) (end 158.5 74.5) (width 0.25) (layer "F.Cu") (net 16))
 (segment (start 160.232613 105.5) (end 154.84 105.5) (width 0.25) (layer "F.Cu") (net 16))
 (segment (start 144.5 74) (end 146.5 74) (width 0.25) (layer "F.Cu") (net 16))
 (segment (start 142.03025 78.207) (end 143.5 76.73725) (width 0.25) (layer "F.Cu") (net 16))
 (segment (start 150 78.5) (end 155.89725 78.5) (width 0.25) (layer "F.Cu") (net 16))
 (segment (start 168.5 80.5) (end 170 82) (width 0.25) (layer "F.Cu") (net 16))
 (segment (start 135.547 78.207) (end 142.03025 78.207) (width 0.25) (layer "F.Cu") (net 16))
 (segment (start 155.89725 78.5) (end 157.5 76.89725) (width 0.25) (layer "F.Cu") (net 16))
 (segment (start 148.12 76.62) (end 150 78.5) (width 0.25) (layer "F.Cu") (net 16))
 (segment (start 154.84 105.5) (end 153.67 106.67) (width 0.25) (layer "F.Cu") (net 16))
 (segment (start 155 108) (end 155 107.88) (width 0.25) (layer "F.Cu") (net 17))
 (segment (start 131.42 76.62) (end 131.42 78.42) (width 0.25) (layer "F.Cu") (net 17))
 (segment (start 134.765 90.964009) (end 134.765 92.265) (width 0.25) (layer "F.Cu") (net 17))
 (segment (start 131.42 87.619009) (end 134.765 90.964009) (width 0.25) (layer "F.Cu") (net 17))
 (segment (start 160.5 101.5) (end 160.5 103) (width 0.25) (layer "F.Cu") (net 17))
 (segment (start 143.2 79) (end 145.58 76.62) (width 0.25) (layer "F.Cu") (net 17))
 (segment (start 160.5 103) (end 159.5 104) (width 0.25) (layer "F.Cu") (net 17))
 (segment (start 140.5 98) (end 157 98) (width 0.25) (layer "F.Cu") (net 17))
 (segment (start 153 108) (end 155 108) (width 0.25) (layer "F.Cu") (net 17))
 (segment (start 131.42 78.42) (end 132 79) (width 0.25) (layer "F.Cu") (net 17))
 (segment (start 157 79) (end 159.5 76.5) (width 0.25) (layer "F.Cu") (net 17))
 (segment (start 157 98) (end 160.5 101.5) (width 0.25) (layer "F.Cu") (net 17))
 (segment (start 154.749009 104) (end 152.5 106.249009) (width 0.25) (layer "F.Cu") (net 17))
 (segment (start 159.5 104) (end 154.749009 104) (width 0.25) (layer "F.Cu") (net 17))
 (segment (start 132 79) (end 143.2 79) (width 0.25) (layer "F.Cu") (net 17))
 (segment (start 131.42 76.62) (end 131.42 87.619009) (width 0.25) (layer "F.Cu") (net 17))
 (segment (start 152.5 106.249009) (end 152.5 107.5) (width 0.25) (layer "F.Cu") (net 17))
 (segment (start 155 107.88) (end 156.21 106.67) (width 0.25) (layer "F.Cu") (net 17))
 (segment (start 134.765 92.265) (end 140.5 98) (width 0.25) (layer "F.Cu") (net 17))
 (segment (start 147.96 79) (end 157 79) (width 0.25) (layer "F.Cu") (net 17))
 (segment (start 145.58 76.62) (end 147.96 79) (width 0.25) (layer "F.Cu") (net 17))
 (segment (start 152.5 107.5) (end 153 108) (width 0.25) (layer "F.Cu") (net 17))
 (segment (start 138.43 89.43) (end 133 84) (width 0.25) (layer "F.Cu") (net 29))
 (segment (start 138.43 91.43) (end 138.43 89.43) (width 0.25) (layer "F.Cu") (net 29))
 (segment (start 124 77) (end 127 80) (width 0.25) (layer "F.Cu") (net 29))
 (segment (start 127 80) (end 127 84) (width 0.25) (layer "F.Cu") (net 29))
 (via (at 133 84) (size 0.8) (drill 0.4) (layers "F.Cu" "B.Cu") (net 29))
 (via (at 127 84) (size 0.8) (drill 0.4) (layers "F.Cu" "B.Cu") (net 29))
 (segment (start 133 84) (end 127 84) (width 0.25) (layer "B.Cu") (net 29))
 (segment (start 122.913 69.587) (end 124 68.5) (width 0.25) (layer "F.Cu") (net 2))
 (segment (start 122.913 86.103) (end 122.913 69.587) (width 0.25) (layer "F.Cu") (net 2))
 (segment (start 125 88.19) (end 123 86.19) (width 0.25) (layer "F.Cu") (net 2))
 (segment (start 125 96.19) (end 125 88.19) (width 0.25) (layer "F.Cu") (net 2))
 (segment (start 123 98.19) (end 125 96.19) (width 0.25) (layer "F.Cu") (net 2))
 (segment (start 163.83 91.43) (end 163.83 89.83) (width 0.25) (layer "B.Cu") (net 2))
 (segment (start 155.74 76.62) (end 147.62 68.5) (width 0.25) (layer "B.Cu") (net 2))
 (segment (start 163.83 89.83) (end 155.74 81.74) (width 0.25) (layer "B.Cu") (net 2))
 (segment (start 147.62 68.5) (end 124 68.5) (width 0.25) (layer "B.Cu") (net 2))
 (segment (start 155.74 81.74) (end 155.74 76.62) (width 0.25) (layer "B.Cu") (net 2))
 (segment (start 169.66 61.26) (end 170.747 62.347) (width 0.25) (layer "F.Cu") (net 11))
 (segment (start 168 64.5) (end 169.66 62.84) (width 0.25) (layer "F.Cu") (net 11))
 (segment (start 170.747 95.622009) (end 160 106.369009) (width 0.25) (layer "F.Cu") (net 11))
 (segment (start 155.74 63.24) (end 157 64.5) (width 0.25) (layer "F.Cu") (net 11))
 (segment (start 143 64.5) (end 154.5 64.5) (width 0.25) (layer "F.Cu") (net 11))
 (segment (start 169.66 62.84) (end 169.66 61.26) (width 0.25) (layer "F.Cu") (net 11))
 (segment (start 157 64.5) (end 168 64.5) (width 0.25) (layer "F.Cu") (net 11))
 (segment (start 141.58 61.38) (end 141.58 63.08) (width 0.25) (layer "F.Cu") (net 11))
 (segment (start 155.74 63.26) (end 155.74 61.38) (width 0.25) (layer "F.Cu") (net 11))
 (segment (start 155.74 63.26) (end 155.74 63.24) (width 0.25) (layer "F.Cu") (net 11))
 (segment (start 142.8 108.5) (end 140.97 106.67) (width 0.25) (layer "F.Cu") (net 11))
 (segment (start 160 106.369009) (end 160 107.010991) (width 0.25) (layer "F.Cu") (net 11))
 (segment (start 141.58 63.08) (end 143 64.5) (width 0.25) (layer "F.Cu") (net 11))
 (segment (start 158.510991 108.5) (end 142.8 108.5) (width 0.25) (layer "F.Cu") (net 11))
 (segment (start 154.5 64.5) (end 155.74 63.26) (width 0.25) (layer "F.Cu") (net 11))
 (segment (start 160 107.010991) (end 158.510991 108.5) (width 0.25) (layer "F.Cu") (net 11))
 (segment (start 170.747 62.347) (end 170.747 95.622009) (width 0.25) (layer "F.Cu") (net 11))
 (segment (start 139.04 61.38) (end 139.04 59.46) (width 0.25) (layer "F.Cu") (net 12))
 (segment (start 141.34 104.5) (end 143.51 106.67) (width 0.25) (layer "F.Cu") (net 12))
 (segment (start 151.5 58) (end 153.2 59.7) (width 0.25) (layer "F.Cu") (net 12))
 (segment (start 165.5 58) (end 167.12 59.62) (width 0.25) (layer "F.Cu") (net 12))
 (segment (start 128.5 58.5) (end 128.5 101.5) (width 0.25) (layer "F.Cu") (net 12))
 (segment (start 139.04 61.38) (end 139.04 59.54) (width 0.25) (layer "F.Cu") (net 12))
 (segment (start 153.2 59.7) (end 153.2 61.38) (width 0.25) (layer "F.Cu") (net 12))
 (segment (start 131.5 104.5) (end 141.34 104.5) (width 0.25) (layer "F.Cu") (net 12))
 (segment (start 139.04 59.54) (end 137.5 58) (width 0.25) (layer "F.Cu") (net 12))
 (segment (start 129 58) (end 128.5 58.5) (width 0.25) (layer "F.Cu") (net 12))
 (segment (start 167.12 59.62) (end 167.12 61.26) (width 0.25) (layer "F.Cu") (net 12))
 (segment (start 128.5 101.5) (end 131.5 104.5) (width 0.25) (layer "F.Cu") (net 12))
 (segment (start 155 58) (end 165.5 58) (width 0.25) (layer "F.Cu") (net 12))
 (segment (start 153.3 59.7) (end 153.2 59.7) (width 0.25) (layer "F.Cu") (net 12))
 (segment (start 155 58) (end 153.3 59.7) (width 0.25) (layer "F.Cu") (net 12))
 (segment (start 139.04 59.46) (end 140.5 58) (width 0.25) (layer "F.Cu") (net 12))
 (segment (start 140.5 58) (end 151.5 58) (width 0.25) (layer "F.Cu") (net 12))
 (segment (start 137.5 58) (end 129 58) (width 0.25) (layer "F.Cu") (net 12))
 (segment (start 150 101) (end 158.5 101) (width 0.25) (layer "F.Cu") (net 13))
 (segment (start 146.05 106.67) (end 146.05 104.95) (width 0.25) (layer "F.Cu") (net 13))
 (segment (start 146.05 104.95) (end 150 101) (width 0.25) (layer "F.Cu") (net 13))
 (via (at 158.5 101) (size 0.8) (drill 0.4) (layers "F.Cu" "B.Cu") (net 13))
 (segment (start 149.5 64.5) (end 160.5 64.5) (width 0.25) (layer "B.Cu") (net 13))
 (segment (start 157.5 73.5) (end 157.5 81) (width 0.25) (layer "B.Cu") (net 13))
 (segment (start 165.245 94.255) (end 158.5 101) (width 0.25) (layer "B.Cu") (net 13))
 (segment (start 133.96 61.38) (end 133.96 62.96) (width 0.25) (layer "B.Cu") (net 13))
 (segment (start 160.5 64.5) (end 162.04 62.96) (width 0.25) (layer "B.Cu") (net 13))
 (segment (start 133.96 62.96) (end 135.5 64.5) (width 0.25) (layer "B.Cu") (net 13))
 (segment (start 165.245 88.745) (end 165.245 94.255) (width 0.25) (layer "B.Cu") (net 13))
 (segment (start 148.12 61.38) (end 148.12 63.12) (width 0.25) (layer "B.Cu") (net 13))
 (segment (start 157.5 81) (end 165.245 88.745) (width 0.25) (layer "B.Cu") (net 13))
 (segment (start 148.12 62.88) (end 148.12 61.38) (width 0.25) (layer "B.Cu") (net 13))
 (segment (start 148.12 63.12) (end 149.5 64.5) (width 0.25) (layer "B.Cu") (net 13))
 (segment (start 148.12 61.38) (end 148.12 64.12) (width 0.25) (layer "B.Cu") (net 13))
 (segment (start 162.04 62.96) (end 162.04 61.26) (width 0.25) (layer "B.Cu") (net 13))
 (segment (start 146.5 64.5) (end 148.12 62.88) (width 0.25) (layer "B.Cu") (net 13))
 (segment (start 135.5 64.5) (end 146.5 64.5) (width 0.25) (layer "B.Cu") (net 13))
 (segment (start 148.12 64.12) (end 157.5 73.5) (width 0.25) (layer "B.Cu") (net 13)))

